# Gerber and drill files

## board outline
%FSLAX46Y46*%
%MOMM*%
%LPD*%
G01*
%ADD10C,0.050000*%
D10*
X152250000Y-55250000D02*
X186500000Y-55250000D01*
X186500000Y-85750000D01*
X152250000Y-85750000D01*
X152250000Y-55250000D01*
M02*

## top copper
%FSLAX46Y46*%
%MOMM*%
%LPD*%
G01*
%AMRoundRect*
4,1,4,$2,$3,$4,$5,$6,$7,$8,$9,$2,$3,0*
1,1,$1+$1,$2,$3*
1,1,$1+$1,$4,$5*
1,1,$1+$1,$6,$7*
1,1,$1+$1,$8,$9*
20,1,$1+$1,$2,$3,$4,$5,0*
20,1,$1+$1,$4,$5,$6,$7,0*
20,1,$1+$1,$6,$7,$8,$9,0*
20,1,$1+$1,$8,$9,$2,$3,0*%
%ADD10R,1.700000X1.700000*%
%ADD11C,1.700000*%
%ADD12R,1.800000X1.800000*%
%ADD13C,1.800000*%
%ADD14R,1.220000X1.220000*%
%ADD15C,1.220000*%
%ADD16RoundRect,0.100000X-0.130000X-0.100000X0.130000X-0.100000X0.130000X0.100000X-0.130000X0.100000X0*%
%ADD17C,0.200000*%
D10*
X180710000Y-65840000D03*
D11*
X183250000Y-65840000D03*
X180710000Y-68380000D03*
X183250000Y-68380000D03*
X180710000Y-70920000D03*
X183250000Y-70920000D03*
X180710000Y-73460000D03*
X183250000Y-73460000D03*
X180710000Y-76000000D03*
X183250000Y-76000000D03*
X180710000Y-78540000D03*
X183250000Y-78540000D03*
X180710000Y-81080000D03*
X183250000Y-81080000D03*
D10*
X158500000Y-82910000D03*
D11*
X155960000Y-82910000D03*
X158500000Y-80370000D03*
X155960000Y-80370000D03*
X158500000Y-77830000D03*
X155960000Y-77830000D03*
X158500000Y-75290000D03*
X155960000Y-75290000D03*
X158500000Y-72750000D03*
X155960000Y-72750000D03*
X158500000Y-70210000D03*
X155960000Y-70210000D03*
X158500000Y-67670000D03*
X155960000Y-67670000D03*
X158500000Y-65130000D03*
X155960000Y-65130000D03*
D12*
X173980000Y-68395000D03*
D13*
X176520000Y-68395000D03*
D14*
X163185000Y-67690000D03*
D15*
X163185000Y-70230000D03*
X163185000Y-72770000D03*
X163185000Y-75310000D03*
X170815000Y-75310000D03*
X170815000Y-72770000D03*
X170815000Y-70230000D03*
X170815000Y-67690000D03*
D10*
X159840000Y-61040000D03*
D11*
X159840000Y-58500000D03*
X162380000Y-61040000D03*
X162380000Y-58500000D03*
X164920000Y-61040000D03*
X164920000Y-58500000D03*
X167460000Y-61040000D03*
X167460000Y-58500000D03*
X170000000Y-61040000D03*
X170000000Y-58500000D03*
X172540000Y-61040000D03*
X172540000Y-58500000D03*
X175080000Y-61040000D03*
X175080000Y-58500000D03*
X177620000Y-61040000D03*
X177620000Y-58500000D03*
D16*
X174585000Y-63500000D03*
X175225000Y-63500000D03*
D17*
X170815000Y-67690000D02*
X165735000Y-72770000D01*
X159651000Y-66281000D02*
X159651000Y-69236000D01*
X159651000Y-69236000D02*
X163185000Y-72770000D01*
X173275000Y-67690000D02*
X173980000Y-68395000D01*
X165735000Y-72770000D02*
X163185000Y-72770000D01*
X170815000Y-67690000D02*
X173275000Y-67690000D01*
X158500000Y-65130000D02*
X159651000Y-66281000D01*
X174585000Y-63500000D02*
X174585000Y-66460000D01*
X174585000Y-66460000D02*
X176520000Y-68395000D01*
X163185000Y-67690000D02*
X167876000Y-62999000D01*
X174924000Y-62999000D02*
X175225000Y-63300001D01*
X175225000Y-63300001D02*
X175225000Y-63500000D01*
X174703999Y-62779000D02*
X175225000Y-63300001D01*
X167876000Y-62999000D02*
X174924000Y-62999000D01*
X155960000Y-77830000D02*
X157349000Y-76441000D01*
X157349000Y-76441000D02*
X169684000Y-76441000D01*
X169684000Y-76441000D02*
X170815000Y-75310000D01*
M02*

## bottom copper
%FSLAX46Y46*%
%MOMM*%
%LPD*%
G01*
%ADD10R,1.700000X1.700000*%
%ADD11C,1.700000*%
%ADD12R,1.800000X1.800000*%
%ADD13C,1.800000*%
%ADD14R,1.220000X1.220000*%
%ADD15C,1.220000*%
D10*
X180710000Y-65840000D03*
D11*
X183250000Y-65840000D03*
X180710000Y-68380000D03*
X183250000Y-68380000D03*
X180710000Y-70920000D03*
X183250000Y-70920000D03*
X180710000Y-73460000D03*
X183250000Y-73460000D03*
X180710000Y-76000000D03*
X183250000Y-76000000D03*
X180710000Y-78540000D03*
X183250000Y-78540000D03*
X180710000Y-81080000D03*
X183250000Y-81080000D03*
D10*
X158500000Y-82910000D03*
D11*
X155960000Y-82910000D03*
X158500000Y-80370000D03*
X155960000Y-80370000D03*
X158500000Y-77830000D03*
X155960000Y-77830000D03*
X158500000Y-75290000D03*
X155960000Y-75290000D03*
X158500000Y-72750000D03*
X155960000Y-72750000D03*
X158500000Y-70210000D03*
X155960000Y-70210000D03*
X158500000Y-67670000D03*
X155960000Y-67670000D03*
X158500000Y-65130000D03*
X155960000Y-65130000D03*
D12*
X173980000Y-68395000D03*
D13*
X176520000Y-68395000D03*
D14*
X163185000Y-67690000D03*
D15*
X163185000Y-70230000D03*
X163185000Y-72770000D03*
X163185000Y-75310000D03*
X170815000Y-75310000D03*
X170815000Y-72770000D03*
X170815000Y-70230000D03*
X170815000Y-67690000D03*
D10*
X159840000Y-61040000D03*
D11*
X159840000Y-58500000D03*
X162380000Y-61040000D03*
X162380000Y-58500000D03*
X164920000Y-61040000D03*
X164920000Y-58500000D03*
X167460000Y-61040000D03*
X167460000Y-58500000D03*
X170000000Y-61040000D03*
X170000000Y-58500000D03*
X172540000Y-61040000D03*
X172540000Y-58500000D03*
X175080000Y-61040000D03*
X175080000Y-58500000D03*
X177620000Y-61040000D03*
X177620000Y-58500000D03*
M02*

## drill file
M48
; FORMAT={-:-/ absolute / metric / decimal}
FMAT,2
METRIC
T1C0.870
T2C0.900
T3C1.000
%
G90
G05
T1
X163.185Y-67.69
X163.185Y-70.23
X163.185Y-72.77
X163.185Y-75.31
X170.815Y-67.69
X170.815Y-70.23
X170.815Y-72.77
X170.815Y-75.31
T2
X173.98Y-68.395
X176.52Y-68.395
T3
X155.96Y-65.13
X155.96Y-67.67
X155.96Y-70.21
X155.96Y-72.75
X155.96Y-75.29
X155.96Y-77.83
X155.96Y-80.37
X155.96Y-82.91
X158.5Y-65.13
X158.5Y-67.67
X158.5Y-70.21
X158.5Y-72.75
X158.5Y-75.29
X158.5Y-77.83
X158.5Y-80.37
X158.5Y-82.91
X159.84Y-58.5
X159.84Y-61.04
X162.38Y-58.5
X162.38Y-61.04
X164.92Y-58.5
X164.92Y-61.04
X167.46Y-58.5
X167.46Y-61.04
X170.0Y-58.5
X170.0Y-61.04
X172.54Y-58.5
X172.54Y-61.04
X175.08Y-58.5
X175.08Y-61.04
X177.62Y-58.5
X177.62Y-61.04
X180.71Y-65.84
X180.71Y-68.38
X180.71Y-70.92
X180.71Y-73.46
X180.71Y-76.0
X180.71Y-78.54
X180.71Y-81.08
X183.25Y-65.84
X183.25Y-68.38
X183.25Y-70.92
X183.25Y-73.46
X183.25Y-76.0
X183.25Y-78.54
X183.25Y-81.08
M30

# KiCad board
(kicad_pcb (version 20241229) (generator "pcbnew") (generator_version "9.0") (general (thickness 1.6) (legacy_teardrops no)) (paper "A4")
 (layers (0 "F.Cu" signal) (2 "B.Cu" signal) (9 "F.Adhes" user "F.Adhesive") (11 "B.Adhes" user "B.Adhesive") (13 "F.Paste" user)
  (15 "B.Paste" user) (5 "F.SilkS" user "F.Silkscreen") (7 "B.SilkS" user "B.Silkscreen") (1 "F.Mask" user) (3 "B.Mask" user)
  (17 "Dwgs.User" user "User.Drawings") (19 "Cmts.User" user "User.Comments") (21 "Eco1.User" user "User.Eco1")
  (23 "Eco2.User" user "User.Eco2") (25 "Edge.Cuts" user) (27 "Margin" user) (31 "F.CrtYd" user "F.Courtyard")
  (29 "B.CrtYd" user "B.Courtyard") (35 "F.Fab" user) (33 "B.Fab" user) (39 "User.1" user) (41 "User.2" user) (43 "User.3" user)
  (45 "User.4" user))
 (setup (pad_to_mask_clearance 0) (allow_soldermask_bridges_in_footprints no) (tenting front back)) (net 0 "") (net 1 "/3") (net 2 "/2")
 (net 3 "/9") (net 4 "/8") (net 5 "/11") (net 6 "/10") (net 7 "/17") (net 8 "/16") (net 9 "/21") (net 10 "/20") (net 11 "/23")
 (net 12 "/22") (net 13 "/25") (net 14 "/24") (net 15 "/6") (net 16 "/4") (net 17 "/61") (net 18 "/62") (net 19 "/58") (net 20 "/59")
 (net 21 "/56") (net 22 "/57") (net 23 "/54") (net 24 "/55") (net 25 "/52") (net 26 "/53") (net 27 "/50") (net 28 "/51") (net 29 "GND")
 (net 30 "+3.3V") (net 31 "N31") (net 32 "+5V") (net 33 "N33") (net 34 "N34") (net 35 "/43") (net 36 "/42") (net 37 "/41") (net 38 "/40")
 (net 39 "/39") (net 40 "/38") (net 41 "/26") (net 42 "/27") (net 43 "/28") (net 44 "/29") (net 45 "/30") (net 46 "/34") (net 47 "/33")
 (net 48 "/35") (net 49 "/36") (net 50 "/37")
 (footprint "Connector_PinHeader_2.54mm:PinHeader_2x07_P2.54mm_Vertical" (layer "F.Cu") (at 180.71 65.84)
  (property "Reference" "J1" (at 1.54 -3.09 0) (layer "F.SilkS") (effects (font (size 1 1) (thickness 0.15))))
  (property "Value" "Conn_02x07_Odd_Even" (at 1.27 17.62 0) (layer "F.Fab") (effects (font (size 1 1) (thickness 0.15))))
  (pad "1" thru_hole rect (at 0 0) (size 1.7 1.7) (drill 1) (layers "*.Cu" "*.Mask") (remove_unused_layers no) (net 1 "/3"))
  (pad "2" thru_hole circle (at 2.54 0) (size 1.7 1.7) (drill 1) (layers "*.Cu" "*.Mask") (remove_unused_layers no) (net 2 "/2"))
  (pad "3" thru_hole circle (at 0 2.54) (size 1.7 1.7) (drill 1) (layers "*.Cu" "*.Mask") (remove_unused_layers no) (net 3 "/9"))
  (pad "4" thru_hole circle (at 2.54 2.54) (size 1.7 1.7) (drill 1) (layers "*.Cu" "*.Mask") (remove_unused_layers no) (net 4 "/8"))
  (pad "5" thru_hole circle (at 0 5.08) (size 1.7 1.7) (drill 1) (layers "*.Cu" "*.Mask") (remove_unused_layers no) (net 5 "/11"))
  (pad "6" thru_hole circle (at 2.54 5.08) (size 1.7 1.7) (drill 1) (layers "*.Cu" "*.Mask") (remove_unused_layers no) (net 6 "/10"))
  (pad "7" thru_hole circle (at 0 7.62) (size 1.7 1.7) (drill 1) (layers "*.Cu" "*.Mask") (remove_unused_layers no) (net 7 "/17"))
  (pad "8" thru_hole circle (at 2.54 7.62) (size 1.7 1.7) (drill 1) (layers "*.Cu" "*.Mask") (remove_unused_layers no) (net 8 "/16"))
  (pad "9" thru_hole circle (at 0 10.16) (size 1.7 1.7) (drill 1) (layers "*.Cu" "*.Mask") (remove_unused_layers no) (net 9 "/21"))
  (pad "10" thru_hole circle (at 2.54 10.16) (size 1.7 1.7) (drill 1) (layers "*.Cu" "*.Mask") (remove_unused_layers no) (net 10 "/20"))
  (pad "11" thru_hole circle (at 0 12.7) (size 1.7 1.7) (drill 1) (layers "*.Cu" "*.Mask") (remove_unused_layers no) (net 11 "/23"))
  (pad "12" thru_hole circle (at 2.54 12.7) (size 1.7 1.7) (drill 1) (layers "*.Cu" "*.Mask") (remove_unused_layers no) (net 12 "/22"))
  (pad "13" thru_hole circle (at 0 15.24) (size 1.7 1.7) (drill 1) (layers "*.Cu" "*.Mask") (remove_unused_layers no) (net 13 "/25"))
  (pad "14" thru_hole circle (at 2.54 15.24) (size 1.7 1.7) (drill 1) (layers "*.Cu" "*.Mask") (remove_unused_layers no) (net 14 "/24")))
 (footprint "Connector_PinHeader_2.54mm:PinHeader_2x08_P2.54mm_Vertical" (layer "F.Cu") (at 158.5 82.91 180)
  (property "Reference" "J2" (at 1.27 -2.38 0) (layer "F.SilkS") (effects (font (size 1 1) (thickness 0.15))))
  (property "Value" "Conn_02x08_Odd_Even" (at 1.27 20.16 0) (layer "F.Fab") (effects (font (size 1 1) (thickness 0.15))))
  (pad "1" thru_hole rect (at 0 0 180) (size 1.7 1.7) (drill 1) (layers "*.Cu" "*.Mask") (remove_unused_layers no) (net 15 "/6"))
  (pad "2" thru_hole circle (at 2.54 0 180) (size 1.7 1.7) (drill 1) (layers "*.Cu" "*.Mask") (remove_unused_layers no) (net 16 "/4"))
  (pad "3" thru_hole circle (at 0 2.54 180) (size 1.7 1.7) (drill 1) (layers "*.Cu" "*.Mask") (remove_unused_layers no) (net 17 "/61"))
  (pad "4" thru_hole circle (at 2.54 2.54 180) (size 1.7 1.7) (drill 1) (layers "*.Cu" "*.Mask") (remove_unused_layers no) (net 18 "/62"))
  (pad "5" thru_hole circle (at 0 5.08 180) (size 1.7 1.7) (drill 1) (layers "*.Cu" "*.Mask") (remove_unused_layers no) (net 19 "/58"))
  (pad "6" thru_hole circle (at 2.54 5.08 180) (size 1.7 1.7) (drill 1) (layers "*.Cu" "*.Mask") (remove_unused_layers no) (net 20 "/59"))
  (pad "7" thru_hole circle (at 0 7.62 180) (size 1.7 1.7) (drill 1) (layers "*.Cu" "*.Mask") (remove_unused_layers no) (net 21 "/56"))
  (pad "8" thru_hole circle (at 2.54 7.62 180) (size 1.7 1.7) (drill 1) (layers "*.Cu" "*.Mask") (remove_unused_layers no) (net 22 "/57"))
  (pad "9" thru_hole circle (at 0 10.16 180) (size 1.7 1.7) (drill 1) (layers "*.Cu" "*.Mask") (remove_unused_layers no) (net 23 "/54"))
  (pad "10" thru_hole circle (at 2.54 10.16 180) (size 1.7 1.7) (drill 1) (layers "*.Cu" "*.Mask") (remove_unused_layers no) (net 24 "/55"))
  (pad "11" thru_hole circle (at 0 12.7 180) (size 1.7 1.7) (drill 1) (layers "*.Cu" "*.Mask") (remove_unused_layers no) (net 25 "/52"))
  (pad "12" thru_hole circle (at 2.54 12.7 180) (size 1.7 1.7) (drill 1) (layers "*.Cu" "*.Mask") (remove_unused_layers no) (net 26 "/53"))
  (pad "13" thru_hole circle (at 0 15.24 180) (size 1.7 1.7) (drill 1) (layers "*.Cu" "*.Mask") (remove_unused_layers no) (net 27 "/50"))
  (pad "14" thru_hole circle (at 2.54 15.24 180) (size 1.7 1.7) (drill 1) (layers "*.Cu" "*.Mask") (remove_unused_layers no) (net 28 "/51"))
  (pad "15" thru_hole circle (at 0 17.78 180) (size 1.7 1.7) (drill 1) (layers "*.Cu" "*.Mask") (remove_unused_layers no) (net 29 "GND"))
  (pad "16" thru_hole circle (at 2.54 17.78 180) (size 1.7 1.7) (drill 1) (layers "*.Cu" "*.Mask") (remove_unused_layers no)
   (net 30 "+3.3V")))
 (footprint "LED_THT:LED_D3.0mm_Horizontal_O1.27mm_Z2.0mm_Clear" (layer "F.Cu") (at 173.98 68.395)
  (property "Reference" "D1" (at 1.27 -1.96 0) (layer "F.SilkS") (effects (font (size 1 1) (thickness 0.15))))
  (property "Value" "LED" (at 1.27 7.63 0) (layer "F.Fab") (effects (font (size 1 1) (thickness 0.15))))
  (pad "1" thru_hole rect (at 0 0) (size 1.8 1.8) (drill 0.9) (layers "*.Cu" "*.Mask") (remove_unused_layers no) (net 29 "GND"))
  (pad "2" thru_hole circle (at 2.54 0) (size 1.8 1.8) (drill 0.9) (layers "*.Cu" "*.Mask") (remove_unused_layers no) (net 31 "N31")))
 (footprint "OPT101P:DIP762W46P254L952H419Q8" (layer "F.Cu") (at 167 71.5)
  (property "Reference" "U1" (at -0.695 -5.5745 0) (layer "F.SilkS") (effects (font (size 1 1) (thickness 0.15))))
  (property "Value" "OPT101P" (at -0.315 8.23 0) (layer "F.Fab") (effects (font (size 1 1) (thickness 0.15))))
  (pad "1" thru_hole rect (at -3.815 -3.81) (size 1.22 1.22) (drill 0.87) (layers "*.Cu" "*.Mask") (remove_unused_layers no) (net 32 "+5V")
   (solder_mask_margin 0.102))
  (pad "2" thru_hole circle (at -3.815 -1.27) (size 1.22 1.22) (drill 0.87) (layers "*.Cu" "*.Mask") (remove_unused_layers no)
   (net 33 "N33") (solder_mask_margin 0.102))
  (pad "3" thru_hole circle (at -3.815 1.27) (size 1.22 1.22) (drill 0.87) (layers "*.Cu" "*.Mask") (remove_unused_layers no) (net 29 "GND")
   (solder_mask_margin 0.102))
  (pad "4" thru_hole circle (at -3.815 3.81) (size 1.22 1.22) (drill 0.87) (layers "*.Cu" "*.Mask") (remove_unused_layers no) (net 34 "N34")
   (solder_mask_margin 0.102))
  (pad "5" thru_hole circle (at 3.815 3.81) (size 1.22 1.22) (drill 0.87) (layers "*.Cu" "*.Mask") (remove_unused_layers no) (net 20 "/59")
   (solder_mask_margin 0.102))
  (pad "6" thru_hole circle (at 3.815 1.27) (size 1.22 1.22) (drill 0.87) (layers "*.Cu" "*.Mask") (remove_unused_layers no)
   (solder_mask_margin 0.102))
  (pad "7" thru_hole circle (at 3.815 -1.27) (size 1.22 1.22) (drill 0.87) (layers "*.Cu" "*.Mask") (remove_unused_layers no)
   (solder_mask_margin 0.102))
  (pad "8" thru_hole circle (at 3.815 -3.81) (size 1.22 1.22) (drill 0.87) (layers "*.Cu" "*.Mask") (remove_unused_layers no) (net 29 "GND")
   (solder_mask_margin 0.102)))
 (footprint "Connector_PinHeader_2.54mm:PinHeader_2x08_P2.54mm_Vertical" (layer "F.Cu") (at 159.84 61.04 90)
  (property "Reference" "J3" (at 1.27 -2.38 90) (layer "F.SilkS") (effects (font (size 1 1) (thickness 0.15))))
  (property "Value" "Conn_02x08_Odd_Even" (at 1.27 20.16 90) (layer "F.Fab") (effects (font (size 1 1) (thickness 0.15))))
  (pad "1" thru_hole rect (at 0 0 90) (size 1.7 1.7) (drill 1) (layers "*.Cu" "*.Mask") (remove_unused_layers no) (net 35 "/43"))
  (pad "2" thru_hole circle (at 2.54 0 90) (size 1.7 1.7) (drill 1) (layers "*.Cu" "*.Mask") (remove_unused_layers no) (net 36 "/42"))
  (pad "3" thru_hole circle (at 0 2.54 90) (size 1.7 1.7) (drill 1) (layers "*.Cu" "*.Mask") (remove_unused_layers no) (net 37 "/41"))
  (pad "4" thru_hole circle (at 2.54 2.54 90) (size 1.7 1.7) (drill 1) (layers "*.Cu" "*.Mask") (remove_unused_layers no) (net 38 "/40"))
  (pad "5" thru_hole circle (at 0 5.08 90) (size 1.7 1.7) (drill 1) (layers "*.Cu" "*.Mask") (remove_unused_layers no) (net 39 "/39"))
  (pad "6" thru_hole circle (at 2.54 5.08 90) (size 1.7 1.7) (drill 1) (layers "*.Cu" "*.Mask") (remove_unused_layers no) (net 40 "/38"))
  (pad "7" thru_hole circle (at 0 7.62 90) (size 1.7 1.7) (drill 1) (layers "*.Cu" "*.Mask") (remove_unused_layers no) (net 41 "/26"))
  (pad "8" thru_hole circle (at 2.54 7.62 90) (size 1.7 1.7) (drill 1) (layers "*.Cu" "*.Mask") (remove_unused_layers no) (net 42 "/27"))
  (pad "9" thru_hole circle (at 0 10.16 90) (size 1.7 1.7) (drill 1) (layers "*.Cu" "*.Mask") (remove_unused_layers no) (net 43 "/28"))
  (pad "10" thru_hole circle (at 2.54 10.16 90) (size 1.7 1.7) (drill 1) (layers "*.Cu" "*.Mask") (remove_unused_layers no) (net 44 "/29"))
  (pad "11" thru_hole circle (at 0 12.7 90) (size 1.7 1.7) (drill 1) (layers "*.Cu" "*.Mask") (remove_unused_layers no) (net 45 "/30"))
  (pad "12" thru_hole circle (at 2.54 12.7 90) (size 1.7 1.7) (drill 1) (layers "*.Cu" "*.Mask") (remove_unused_layers no) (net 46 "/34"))
  (pad "13" thru_hole circle (at 0 15.24 90) (size 1.7 1.7) (drill 1) (layers "*.Cu" "*.Mask") (remove_unused_layers no) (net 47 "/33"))
  (pad "14" thru_hole circle (at 2.54 15.24 90) (size 1.7 1.7) (drill 1) (layers "*.Cu" "*.Mask") (remove_unused_layers no) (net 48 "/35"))
  (pad "15" thru_hole circle (at 0 17.78 90) (size 1.7 1.7) (drill 1) (layers "*.Cu" "*.Mask") (remove_unused_layers no) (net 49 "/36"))
  (pad "16" thru_hole circle (at 2.54 17.78 90) (size 1.7 1.7) (drill 1) (layers "*.Cu" "*.Mask") (remove_unused_layers no) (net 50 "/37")))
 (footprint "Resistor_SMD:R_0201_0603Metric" (layer "F.Cu") (at 174.905 63.5)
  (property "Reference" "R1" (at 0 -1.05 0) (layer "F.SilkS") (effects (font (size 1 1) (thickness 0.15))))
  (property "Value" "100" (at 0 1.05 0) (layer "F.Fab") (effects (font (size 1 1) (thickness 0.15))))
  (pad "" smd roundrect (at -0.345 0) (size 0.318 0.36) (layers "F.Paste") (roundrect_rratio 0.25))
  (pad "" smd roundrect (at 0.345 0) (size 0.318 0.36) (layers "F.Paste") (roundrect_rratio 0.25))
  (pad "1" smd roundrect (at -0.32 0) (size 0.46 0.4) (layers "F.Cu" "F.Mask") (roundrect_rratio 0.25) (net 31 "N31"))
  (pad "2" smd roundrect (at 0.32 0) (size 0.46 0.4) (layers "F.Cu" "F.Mask") (roundrect_rratio 0.25) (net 32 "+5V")))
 (gr_rect (start 152.25 55.25) (end 186.5 85.75) (stroke (width 0.05) (type default)) (fill no) (layer "Edge.Cuts"))
 (segment (start 170.815 67.69) (end 165.735 72.77) (width 0.2) (layer "F.Cu") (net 29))
 (segment (start 159.651 66.281) (end 159.651 69.236) (width 0.2) (layer "F.Cu") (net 29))
 (segment (start 159.651 69.236) (end 163.185 72.77) (width 0.2) (layer "F.Cu") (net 29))
 (segment (start 173.275 67.69) (end 173.98 68.395) (width 0.2) (layer "F.Cu") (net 29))
 (segment (start 165.735 72.77) (end 163.185 72.77) (width 0.2) (layer "F.Cu") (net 29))
 (segment (start 170.815 67.69) (end 173.275 67.69) (width 0.2) (layer "F.Cu") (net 29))
 (segment (start 158.5 65.13) (end 159.651 66.281) (width 0.2) (layer "F.Cu") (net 29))
 (segment (start 174.585 63.5) (end 174.585 66.46) (width 0.2) (layer "F.Cu") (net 31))
 (segment (start 174.585 66.46) (end 176.52 68.395) (width 0.2) (layer "F.Cu") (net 31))
 (segment (start 163.185 67.69) (end 167.876 62.999) (width 0.2) (layer "F.Cu") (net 32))
 (segment (start 174.924 62.999) (end 175.225 63.300001) (width 0.2) (layer "F.Cu") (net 32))
 (segment (start 175.225 63.300001) (end 175.225 63.5) (width 0.2) (layer "F.Cu") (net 32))
 (segment (start 174.703999 62.779) (end 175.225 63.300001) (width 0.2) (layer "F.Cu") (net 32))
 (segment (start 167.876 62.999) (end 174.924 62.999) (width 0.2) (layer "F.Cu") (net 32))
 (segment (start 155.96 77.83) (end 157.349 76.441) (width 0.2) (layer "F.Cu") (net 20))
 (segment (start 157.349 76.441) (end 169.684 76.441) (width 0.2) (layer "F.Cu") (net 20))
 (segment (start 169.684 76.441) (end 170.815 75.31) (width 0.2) (layer "F.Cu") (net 20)))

